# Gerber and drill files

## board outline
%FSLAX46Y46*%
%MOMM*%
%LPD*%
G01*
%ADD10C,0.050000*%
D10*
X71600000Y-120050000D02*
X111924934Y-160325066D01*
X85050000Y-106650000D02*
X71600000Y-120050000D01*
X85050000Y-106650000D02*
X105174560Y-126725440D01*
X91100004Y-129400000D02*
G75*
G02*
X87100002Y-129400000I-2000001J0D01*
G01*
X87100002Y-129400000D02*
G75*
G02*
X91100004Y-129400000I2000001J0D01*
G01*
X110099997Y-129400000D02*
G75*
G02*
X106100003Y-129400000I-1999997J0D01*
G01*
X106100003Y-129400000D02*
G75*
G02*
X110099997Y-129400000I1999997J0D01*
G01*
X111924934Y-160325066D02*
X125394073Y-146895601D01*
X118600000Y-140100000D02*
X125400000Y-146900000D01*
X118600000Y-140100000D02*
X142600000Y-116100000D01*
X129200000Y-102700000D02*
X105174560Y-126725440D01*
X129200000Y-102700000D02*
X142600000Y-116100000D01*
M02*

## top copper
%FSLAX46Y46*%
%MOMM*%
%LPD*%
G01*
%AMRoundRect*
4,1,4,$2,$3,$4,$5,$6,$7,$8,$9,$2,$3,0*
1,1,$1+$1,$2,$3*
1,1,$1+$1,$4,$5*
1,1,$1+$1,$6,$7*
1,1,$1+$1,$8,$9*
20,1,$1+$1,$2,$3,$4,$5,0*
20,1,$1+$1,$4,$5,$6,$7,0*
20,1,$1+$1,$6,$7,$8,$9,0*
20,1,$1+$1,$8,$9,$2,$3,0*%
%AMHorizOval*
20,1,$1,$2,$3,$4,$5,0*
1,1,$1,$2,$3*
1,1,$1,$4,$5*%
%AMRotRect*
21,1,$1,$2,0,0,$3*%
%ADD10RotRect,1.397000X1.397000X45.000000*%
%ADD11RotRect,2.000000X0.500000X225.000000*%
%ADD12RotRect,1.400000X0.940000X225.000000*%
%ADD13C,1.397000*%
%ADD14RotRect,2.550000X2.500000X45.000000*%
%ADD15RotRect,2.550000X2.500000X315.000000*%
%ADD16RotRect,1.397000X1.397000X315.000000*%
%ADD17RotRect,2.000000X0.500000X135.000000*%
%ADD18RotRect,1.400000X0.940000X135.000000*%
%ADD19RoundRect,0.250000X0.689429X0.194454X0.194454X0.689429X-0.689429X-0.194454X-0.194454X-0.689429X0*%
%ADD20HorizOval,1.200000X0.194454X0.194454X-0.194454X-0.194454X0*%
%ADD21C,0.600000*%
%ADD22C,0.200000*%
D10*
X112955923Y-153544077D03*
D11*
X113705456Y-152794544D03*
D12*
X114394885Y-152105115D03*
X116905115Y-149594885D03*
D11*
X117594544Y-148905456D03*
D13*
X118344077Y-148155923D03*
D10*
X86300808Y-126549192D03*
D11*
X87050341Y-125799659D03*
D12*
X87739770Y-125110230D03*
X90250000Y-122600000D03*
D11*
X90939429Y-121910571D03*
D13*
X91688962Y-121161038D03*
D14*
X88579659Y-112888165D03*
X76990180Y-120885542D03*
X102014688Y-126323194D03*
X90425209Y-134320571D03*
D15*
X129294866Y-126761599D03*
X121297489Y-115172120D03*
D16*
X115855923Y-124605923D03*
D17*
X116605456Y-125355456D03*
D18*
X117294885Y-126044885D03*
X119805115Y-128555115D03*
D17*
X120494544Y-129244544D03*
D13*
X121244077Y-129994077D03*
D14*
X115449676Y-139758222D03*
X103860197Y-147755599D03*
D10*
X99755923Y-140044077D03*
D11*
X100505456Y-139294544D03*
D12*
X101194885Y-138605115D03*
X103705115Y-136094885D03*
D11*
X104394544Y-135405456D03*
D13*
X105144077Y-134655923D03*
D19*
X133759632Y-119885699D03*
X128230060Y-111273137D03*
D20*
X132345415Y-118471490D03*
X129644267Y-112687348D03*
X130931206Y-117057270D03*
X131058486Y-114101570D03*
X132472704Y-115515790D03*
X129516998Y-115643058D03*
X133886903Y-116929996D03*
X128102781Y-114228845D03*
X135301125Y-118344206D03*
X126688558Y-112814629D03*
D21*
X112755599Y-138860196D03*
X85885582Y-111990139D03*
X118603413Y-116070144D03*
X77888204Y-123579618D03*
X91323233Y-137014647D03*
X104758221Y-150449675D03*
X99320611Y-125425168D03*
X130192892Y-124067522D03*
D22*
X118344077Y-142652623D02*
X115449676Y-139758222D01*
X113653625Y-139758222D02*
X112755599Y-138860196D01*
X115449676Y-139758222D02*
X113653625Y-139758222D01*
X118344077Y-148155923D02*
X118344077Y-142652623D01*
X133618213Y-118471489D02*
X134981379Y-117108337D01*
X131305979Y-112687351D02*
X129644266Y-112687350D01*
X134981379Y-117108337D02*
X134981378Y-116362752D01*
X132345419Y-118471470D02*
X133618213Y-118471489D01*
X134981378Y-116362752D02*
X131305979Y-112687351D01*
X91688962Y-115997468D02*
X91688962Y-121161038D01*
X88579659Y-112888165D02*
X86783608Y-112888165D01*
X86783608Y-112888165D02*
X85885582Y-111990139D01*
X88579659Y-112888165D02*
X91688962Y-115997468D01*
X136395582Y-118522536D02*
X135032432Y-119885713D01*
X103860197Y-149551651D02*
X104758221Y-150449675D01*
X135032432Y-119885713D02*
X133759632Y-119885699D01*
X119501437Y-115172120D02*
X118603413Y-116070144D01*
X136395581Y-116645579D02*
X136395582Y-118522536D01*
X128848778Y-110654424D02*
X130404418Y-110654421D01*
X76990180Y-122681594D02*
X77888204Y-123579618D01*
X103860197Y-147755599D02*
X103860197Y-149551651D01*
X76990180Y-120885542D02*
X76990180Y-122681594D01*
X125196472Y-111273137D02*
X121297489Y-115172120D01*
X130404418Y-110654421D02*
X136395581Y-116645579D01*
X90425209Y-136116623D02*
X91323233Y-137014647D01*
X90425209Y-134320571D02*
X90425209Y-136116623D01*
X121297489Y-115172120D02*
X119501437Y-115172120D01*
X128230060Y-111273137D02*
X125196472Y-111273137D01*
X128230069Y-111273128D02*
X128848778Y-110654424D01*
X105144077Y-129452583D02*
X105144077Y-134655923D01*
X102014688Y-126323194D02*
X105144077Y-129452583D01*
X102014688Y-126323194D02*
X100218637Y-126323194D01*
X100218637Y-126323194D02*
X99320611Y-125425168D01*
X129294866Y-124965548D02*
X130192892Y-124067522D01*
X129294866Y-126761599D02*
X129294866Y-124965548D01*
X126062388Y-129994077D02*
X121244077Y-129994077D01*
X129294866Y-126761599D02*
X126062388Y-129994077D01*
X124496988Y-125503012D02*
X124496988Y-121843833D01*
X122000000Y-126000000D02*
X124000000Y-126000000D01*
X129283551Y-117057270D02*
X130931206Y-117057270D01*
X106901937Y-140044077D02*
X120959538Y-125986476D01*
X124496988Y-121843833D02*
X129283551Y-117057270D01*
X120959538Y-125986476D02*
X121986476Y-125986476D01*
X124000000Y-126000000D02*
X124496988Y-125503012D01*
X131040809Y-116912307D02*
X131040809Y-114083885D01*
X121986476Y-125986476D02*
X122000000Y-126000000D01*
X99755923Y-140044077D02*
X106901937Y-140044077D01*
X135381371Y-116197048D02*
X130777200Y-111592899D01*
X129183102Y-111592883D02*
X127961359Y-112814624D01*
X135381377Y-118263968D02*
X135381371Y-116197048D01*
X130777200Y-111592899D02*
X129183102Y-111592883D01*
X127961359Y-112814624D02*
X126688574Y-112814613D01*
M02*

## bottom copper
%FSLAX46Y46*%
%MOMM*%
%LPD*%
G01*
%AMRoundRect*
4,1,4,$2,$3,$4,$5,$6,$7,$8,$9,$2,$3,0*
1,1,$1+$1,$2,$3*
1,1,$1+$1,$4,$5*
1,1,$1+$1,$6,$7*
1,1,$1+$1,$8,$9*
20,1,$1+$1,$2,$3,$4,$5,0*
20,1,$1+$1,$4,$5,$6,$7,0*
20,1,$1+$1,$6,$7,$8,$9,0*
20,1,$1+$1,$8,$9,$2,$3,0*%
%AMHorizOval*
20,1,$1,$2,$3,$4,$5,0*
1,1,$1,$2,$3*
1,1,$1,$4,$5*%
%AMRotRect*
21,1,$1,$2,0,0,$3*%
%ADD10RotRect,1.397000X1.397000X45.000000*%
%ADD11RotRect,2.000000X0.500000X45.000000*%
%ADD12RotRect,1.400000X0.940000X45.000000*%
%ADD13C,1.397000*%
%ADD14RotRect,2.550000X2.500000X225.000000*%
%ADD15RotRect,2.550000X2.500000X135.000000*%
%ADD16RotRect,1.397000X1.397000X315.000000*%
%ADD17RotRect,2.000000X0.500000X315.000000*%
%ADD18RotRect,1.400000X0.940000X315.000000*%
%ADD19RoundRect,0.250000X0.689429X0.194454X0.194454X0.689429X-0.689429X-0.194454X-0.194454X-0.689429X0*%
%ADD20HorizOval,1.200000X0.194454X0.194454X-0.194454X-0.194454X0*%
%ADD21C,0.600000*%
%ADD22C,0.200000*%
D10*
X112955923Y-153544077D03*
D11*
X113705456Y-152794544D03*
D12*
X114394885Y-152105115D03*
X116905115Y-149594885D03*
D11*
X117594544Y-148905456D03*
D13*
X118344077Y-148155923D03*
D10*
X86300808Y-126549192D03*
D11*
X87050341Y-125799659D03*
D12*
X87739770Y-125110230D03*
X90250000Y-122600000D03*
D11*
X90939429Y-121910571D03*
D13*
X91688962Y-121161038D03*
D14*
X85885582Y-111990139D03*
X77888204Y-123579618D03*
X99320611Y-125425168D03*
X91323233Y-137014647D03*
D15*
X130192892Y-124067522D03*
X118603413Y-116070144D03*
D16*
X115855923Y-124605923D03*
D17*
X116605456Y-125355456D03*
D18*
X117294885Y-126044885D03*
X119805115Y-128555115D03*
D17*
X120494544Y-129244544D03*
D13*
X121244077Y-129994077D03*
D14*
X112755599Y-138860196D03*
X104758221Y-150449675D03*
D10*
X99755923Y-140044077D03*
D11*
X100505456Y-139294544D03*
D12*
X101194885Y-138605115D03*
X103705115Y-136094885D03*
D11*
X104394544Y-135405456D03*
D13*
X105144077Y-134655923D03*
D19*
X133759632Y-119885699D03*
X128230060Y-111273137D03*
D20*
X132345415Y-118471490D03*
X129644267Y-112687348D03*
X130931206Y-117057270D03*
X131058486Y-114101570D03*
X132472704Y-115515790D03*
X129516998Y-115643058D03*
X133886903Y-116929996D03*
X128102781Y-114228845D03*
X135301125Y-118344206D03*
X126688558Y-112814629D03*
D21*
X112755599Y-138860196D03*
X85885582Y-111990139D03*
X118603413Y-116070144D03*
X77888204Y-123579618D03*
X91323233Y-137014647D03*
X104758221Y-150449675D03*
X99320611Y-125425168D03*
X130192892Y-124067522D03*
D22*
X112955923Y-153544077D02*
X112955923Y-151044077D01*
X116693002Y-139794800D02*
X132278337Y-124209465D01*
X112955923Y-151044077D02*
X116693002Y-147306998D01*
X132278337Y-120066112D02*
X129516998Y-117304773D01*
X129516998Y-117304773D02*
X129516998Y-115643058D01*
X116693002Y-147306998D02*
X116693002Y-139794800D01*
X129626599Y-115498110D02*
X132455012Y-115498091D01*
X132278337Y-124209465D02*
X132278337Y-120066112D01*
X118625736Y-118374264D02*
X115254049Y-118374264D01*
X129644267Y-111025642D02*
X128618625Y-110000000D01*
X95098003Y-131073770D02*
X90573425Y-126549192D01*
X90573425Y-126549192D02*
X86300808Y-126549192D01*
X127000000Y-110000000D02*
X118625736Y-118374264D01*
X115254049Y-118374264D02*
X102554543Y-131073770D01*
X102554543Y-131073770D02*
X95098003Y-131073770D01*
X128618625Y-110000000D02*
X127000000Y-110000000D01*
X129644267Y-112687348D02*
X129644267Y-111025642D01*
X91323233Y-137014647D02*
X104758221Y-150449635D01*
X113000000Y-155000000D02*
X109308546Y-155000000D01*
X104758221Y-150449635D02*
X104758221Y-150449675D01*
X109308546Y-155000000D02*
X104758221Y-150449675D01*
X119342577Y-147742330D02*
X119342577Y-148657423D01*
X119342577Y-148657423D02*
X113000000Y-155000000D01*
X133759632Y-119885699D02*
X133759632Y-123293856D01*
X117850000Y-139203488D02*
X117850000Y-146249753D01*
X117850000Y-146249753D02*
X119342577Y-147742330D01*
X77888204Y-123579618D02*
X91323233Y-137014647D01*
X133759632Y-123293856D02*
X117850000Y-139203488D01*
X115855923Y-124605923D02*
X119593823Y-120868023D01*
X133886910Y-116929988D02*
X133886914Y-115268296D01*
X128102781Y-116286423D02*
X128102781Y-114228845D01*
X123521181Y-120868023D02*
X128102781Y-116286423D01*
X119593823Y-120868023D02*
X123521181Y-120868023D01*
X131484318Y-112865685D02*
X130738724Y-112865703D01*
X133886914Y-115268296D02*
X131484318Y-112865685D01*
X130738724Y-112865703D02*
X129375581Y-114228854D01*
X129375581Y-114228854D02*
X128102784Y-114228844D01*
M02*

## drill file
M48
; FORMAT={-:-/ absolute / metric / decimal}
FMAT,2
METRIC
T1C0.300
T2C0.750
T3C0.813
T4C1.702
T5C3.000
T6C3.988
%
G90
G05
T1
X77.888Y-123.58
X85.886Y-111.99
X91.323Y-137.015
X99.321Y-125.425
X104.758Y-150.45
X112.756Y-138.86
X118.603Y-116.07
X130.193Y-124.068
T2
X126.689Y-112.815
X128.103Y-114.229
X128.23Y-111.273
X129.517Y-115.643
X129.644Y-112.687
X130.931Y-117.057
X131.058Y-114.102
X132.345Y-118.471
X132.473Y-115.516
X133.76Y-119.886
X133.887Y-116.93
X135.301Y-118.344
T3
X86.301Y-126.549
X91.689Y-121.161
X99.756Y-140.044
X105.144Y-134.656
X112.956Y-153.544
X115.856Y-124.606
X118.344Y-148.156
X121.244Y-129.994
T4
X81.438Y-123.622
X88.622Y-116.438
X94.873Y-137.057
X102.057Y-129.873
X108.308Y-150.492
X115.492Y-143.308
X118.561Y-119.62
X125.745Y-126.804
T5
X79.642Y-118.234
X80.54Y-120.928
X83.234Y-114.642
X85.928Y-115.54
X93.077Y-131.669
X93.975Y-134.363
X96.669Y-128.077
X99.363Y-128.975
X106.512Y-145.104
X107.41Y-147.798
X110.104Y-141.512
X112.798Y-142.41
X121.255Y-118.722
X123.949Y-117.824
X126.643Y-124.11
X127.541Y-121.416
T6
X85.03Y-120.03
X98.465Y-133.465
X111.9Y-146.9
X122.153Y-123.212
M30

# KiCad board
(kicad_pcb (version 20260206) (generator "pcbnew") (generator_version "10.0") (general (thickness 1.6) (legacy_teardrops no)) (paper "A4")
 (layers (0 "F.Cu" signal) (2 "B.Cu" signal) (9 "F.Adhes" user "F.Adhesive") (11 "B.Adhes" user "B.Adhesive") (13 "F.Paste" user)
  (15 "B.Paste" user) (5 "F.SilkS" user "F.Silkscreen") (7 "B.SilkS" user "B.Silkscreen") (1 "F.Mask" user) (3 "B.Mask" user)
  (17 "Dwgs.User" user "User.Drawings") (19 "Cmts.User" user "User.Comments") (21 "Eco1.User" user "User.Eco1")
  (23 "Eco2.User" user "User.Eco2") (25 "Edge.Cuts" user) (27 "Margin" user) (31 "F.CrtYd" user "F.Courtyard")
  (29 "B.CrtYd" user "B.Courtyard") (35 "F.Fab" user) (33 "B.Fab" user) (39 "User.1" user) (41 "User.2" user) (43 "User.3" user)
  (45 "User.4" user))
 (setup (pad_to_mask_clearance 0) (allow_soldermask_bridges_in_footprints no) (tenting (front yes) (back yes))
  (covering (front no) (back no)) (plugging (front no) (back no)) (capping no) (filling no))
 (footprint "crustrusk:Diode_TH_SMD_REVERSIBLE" (layer "F.Cu") (at 115.65 150.85 45)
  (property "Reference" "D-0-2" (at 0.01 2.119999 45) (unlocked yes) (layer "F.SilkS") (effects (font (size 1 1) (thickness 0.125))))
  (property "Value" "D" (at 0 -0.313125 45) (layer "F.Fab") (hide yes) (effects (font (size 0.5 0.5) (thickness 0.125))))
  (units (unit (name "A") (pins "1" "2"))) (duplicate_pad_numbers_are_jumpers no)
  (pad "1" thru_hole rect (at -3.81 0 45) (size 1.397 1.397) (drill 0.8128) (layers "*.Cu" "*.Mask") (remove_unused_layers no)
   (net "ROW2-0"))
  (pad "1" smd rect (at -2.75 0 225) (size 2 0.5) (layers "F.Cu") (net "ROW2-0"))
  (pad "1" smd rect (at -2.75 0 45) (size 2 0.5) (layers "B.Cu") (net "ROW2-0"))
  (pad "1" smd rect (at -1.775001 0 225) (size 1.4 0.94) (layers "F.Cu" "F.Mask" "F.Paste") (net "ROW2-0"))
  (pad "1" smd rect (at -1.775001 0 45) (size 1.4 0.94) (layers "B.Cu" "B.Mask" "B.Paste") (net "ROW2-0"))
  (pad "2" smd rect (at 1.775001 0 225) (size 1.4 0.94) (layers "F.Cu" "F.Mask" "F.Paste") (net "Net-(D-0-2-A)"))
  (pad "2" smd rect (at 1.775001 0 45) (size 1.4 0.94) (layers "B.Cu" "B.Mask" "B.Paste") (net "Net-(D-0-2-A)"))
  (pad "2" smd rect (at 2.75 0 225) (size 2 0.5) (layers "F.Cu") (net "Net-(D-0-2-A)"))
  (pad "2" smd rect (at 2.75 0 45) (size 2 0.5) (layers "B.Cu") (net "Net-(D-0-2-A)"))
  (pad "2" thru_hole circle (at 3.81 0 45) (size 1.397 1.397) (drill 0.8128) (layers "*.Cu" "*.Mask") (remove_unused_layers no)
   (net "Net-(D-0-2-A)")))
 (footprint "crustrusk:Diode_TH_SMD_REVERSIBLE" (layer "F.Cu") (at 88.994885 123.855115 45)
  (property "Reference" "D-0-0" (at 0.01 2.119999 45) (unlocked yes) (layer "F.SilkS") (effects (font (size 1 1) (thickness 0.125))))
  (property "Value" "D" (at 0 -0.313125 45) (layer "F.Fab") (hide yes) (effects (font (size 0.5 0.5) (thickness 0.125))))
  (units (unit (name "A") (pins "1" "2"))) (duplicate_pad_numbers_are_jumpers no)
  (pad "1" thru_hole rect (at -3.81 0 45) (size 1.397 1.397) (drill 0.8128) (layers "*.Cu" "*.Mask") (remove_unused_layers no)
   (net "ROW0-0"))
  (pad "1" smd rect (at -2.75 0 225) (size 2 0.5) (layers "F.Cu") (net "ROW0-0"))
  (pad "1" smd rect (at -2.75 0 45) (size 2 0.5) (layers "B.Cu") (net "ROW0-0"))
  (pad "1" smd rect (at -1.775001 0 225) (size 1.4 0.94) (layers "F.Cu" "F.Mask" "F.Paste") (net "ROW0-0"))
  (pad "1" smd rect (at -1.775001 0 45) (size 1.4 0.94) (layers "B.Cu" "B.Mask" "B.Paste") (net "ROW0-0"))
  (pad "2" smd rect (at 1.775001 0 225) (size 1.4 0.94) (layers "F.Cu" "F.Mask" "F.Paste") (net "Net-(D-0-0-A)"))
  (pad "2" smd rect (at 1.775001 0 45) (size 1.4 0.94) (layers "B.Cu" "B.Mask" "B.Paste") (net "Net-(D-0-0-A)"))
  (pad "2" smd rect (at 2.75 0 225) (size 2 0.5) (layers "F.Cu") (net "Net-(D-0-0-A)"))
  (pad "2" smd rect (at 2.75 0 45) (size 2 0.5) (layers "B.Cu") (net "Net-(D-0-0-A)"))
  (pad "2" thru_hole circle (at 3.81 0 45) (size 1.397 1.397) (drill 0.8128) (layers "*.Cu" "*.Mask") (remove_unused_layers no)
   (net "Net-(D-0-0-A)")))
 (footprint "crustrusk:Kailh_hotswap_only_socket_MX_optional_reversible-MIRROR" (layer "F.Cu") (at 85.029983 120.029943 45)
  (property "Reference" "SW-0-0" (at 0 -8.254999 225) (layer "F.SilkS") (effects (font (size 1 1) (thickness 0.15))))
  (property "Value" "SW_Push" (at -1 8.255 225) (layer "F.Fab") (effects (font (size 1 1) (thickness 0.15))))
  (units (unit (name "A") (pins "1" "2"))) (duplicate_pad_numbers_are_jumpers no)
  (pad "" np_thru_hole circle (at -5.079999 0 45) (size 1.7018 1.7018) (drill 1.7018) (layers "*.Cu" "*.Mask"))
  (pad "" np_thru_hole circle (at -3.81 -2.54 225) (size 3 3) (drill 3) (layers "*.Cu" "*.Mask"))
  (pad "" np_thru_hole circle (at -2.54 -5.079998 45) (size 3 3) (drill 3) (layers "*.Cu" "*.Mask"))
  (pad "" np_thru_hole circle (at 0 0 45) (size 3.9878 3.9878) (drill 3.9878) (layers "*.Cu" "*.Mask"))
  (pad "" np_thru_hole circle (at 2.540002 -5.080001 225) (size 3 3) (drill 3) (layers "*.Cu" "*.Mask"))
  (pad "" np_thru_hole circle (at 3.81 -2.54 45) (size 3 3) (drill 3) (layers "*.Cu" "*.Mask"))
  (pad "" np_thru_hole circle (at 5.079999 0 45) (size 1.7018 1.7018) (drill 1.7018) (layers "*.Cu" "*.Mask"))
  (pad "1" smd rect (at 6.29 -5.08 225) (size 2.55 2.5) (layers "B.Cu" "B.Mask" "B.Paste") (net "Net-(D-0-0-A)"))
  (pad "1" smd rect (at 7.56 -2.54 45) (size 2.55 2.5) (layers "F.Cu" "F.Mask" "F.Paste") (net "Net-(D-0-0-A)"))
  (pad "2" smd rect (at -7.56 -2.540001 225) (size 2.55 2.5) (layers "B.Cu" "B.Mask" "B.Paste") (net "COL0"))
  (pad "2" smd rect (at -6.289999 -5.079999 45) (size 2.55 2.5) (layers "F.Cu" "F.Mask" "F.Paste") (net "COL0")))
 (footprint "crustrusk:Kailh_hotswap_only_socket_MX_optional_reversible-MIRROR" (layer "F.Cu") (at 98.465012 133.464972 45)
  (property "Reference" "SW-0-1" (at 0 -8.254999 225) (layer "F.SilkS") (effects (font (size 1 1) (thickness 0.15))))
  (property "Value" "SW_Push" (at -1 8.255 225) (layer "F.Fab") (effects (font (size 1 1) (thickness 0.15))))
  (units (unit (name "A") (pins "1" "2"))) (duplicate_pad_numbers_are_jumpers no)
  (pad "" np_thru_hole circle (at -5.079999 0 45) (size 1.7018 1.7018) (drill 1.7018) (layers "*.Cu" "*.Mask"))
  (pad "" np_thru_hole circle (at -3.81 -2.54 225) (size 3 3) (drill 3) (layers "*.Cu" "*.Mask"))
  (pad "" np_thru_hole circle (at -2.54 -5.079998 45) (size 3 3) (drill 3) (layers "*.Cu" "*.Mask"))
  (pad "" np_thru_hole circle (at 0 0 45) (size 3.9878 3.9878) (drill 3.9878) (layers "*.Cu" "*.Mask"))
  (pad "" np_thru_hole circle (at 2.540002 -5.080001 225) (size 3 3) (drill 3) (layers "*.Cu" "*.Mask"))
  (pad "" np_thru_hole circle (at 3.81 -2.54 45) (size 3 3) (drill 3) (layers "*.Cu" "*.Mask"))
  (pad "" np_thru_hole circle (at 5.079999 0 45) (size 1.7018 1.7018) (drill 1.7018) (layers "*.Cu" "*.Mask"))
  (pad "1" smd rect (at 6.29 -5.08 225) (size 2.55 2.5) (layers "B.Cu" "B.Mask" "B.Paste") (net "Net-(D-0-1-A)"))
  (pad "1" smd rect (at 7.56 -2.54 45) (size 2.55 2.5) (layers "F.Cu" "F.Mask" "F.Paste") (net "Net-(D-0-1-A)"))
  (pad "2" smd rect (at -7.56 -2.540001 225) (size 2.55 2.5) (layers "B.Cu" "B.Mask" "B.Paste") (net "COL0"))
  (pad "2" smd rect (at -6.289999 -5.079999 45) (size 2.55 2.5) (layers "F.Cu" "F.Mask" "F.Paste") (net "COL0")))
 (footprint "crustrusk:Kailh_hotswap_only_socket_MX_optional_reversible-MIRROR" (layer "F.Cu") (at 122.153088 123.211923 -45)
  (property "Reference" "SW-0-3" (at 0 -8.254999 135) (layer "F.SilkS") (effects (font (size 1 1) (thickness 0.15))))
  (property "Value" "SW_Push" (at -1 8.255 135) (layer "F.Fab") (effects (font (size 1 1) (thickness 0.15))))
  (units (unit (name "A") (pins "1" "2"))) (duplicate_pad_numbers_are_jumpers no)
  (pad "" np_thru_hole circle (at -5.079999 0 315) (size 1.7018 1.7018) (drill 1.7018) (layers "*.Cu" "*.Mask"))
  (pad "" np_thru_hole circle (at -3.81 -2.54 135) (size 3 3) (drill 3) (layers "*.Cu" "*.Mask"))
  (pad "" np_thru_hole circle (at -2.54 -5.079998 315) (size 3 3) (drill 3) (layers "*.Cu" "*.Mask"))
  (pad "" np_thru_hole circle (at 0 0 315) (size 3.9878 3.9878) (drill 3.9878) (layers "*.Cu" "*.Mask"))
  (pad "" np_thru_hole circle (at 2.540002 -5.080001 135) (size 3 3) (drill 3) (layers "*.Cu" "*.Mask"))
  (pad "" np_thru_hole circle (at 3.81 -2.54 315) (size 3 3) (drill 3) (layers "*.Cu" "*.Mask"))
  (pad "" np_thru_hole circle (at 5.079999 0 315) (size 1.7018 1.7018) (drill 1.7018) (layers "*.Cu" "*.Mask"))
  (pad "1" smd rect (at 6.29 -5.08 135) (size 2.55 2.5) (layers "B.Cu" "B.Mask" "B.Paste") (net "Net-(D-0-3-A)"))
  (pad "1" smd rect (at 7.56 -2.54 315) (size 2.55 2.5) (layers "F.Cu" "F.Mask" "F.Paste") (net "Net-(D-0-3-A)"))
  (pad "2" smd rect (at -7.56 -2.540001 135) (size 2.55 2.5) (layers "B.Cu" "B.Mask" "B.Paste") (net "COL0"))
  (pad "2" smd rect (at -6.289999 -5.079999 315) (size 2.55 2.5) (layers "F.Cu" "F.Mask" "F.Paste") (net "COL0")))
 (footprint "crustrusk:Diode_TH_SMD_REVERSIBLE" (layer "F.Cu") (at 118.55 127.3 -45)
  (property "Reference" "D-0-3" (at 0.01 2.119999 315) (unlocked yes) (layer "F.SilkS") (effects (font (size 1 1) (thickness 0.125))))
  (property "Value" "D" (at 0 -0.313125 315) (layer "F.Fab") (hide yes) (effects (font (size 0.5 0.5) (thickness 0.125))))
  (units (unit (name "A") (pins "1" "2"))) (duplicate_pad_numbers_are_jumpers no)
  (pad "1" thru_hole rect (at -3.81 0 315) (size 1.397 1.397) (drill 0.8128) (layers "*.Cu" "*.Mask") (remove_unused_layers no)
   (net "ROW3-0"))
  (pad "1" smd rect (at -2.75 0 135) (size 2 0.5) (layers "F.Cu") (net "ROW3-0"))
  (pad "1" smd rect (at -2.75 0 315) (size 2 0.5) (layers "B.Cu") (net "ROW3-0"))
  (pad "1" smd rect (at -1.775001 0 135) (size 1.4 0.94) (layers "F.Cu" "F.Mask" "F.Paste") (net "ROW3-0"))
  (pad "1" smd rect (at -1.775001 0 315) (size 1.4 0.94) (layers "B.Cu" "B.Mask" "B.Paste") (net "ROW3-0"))
  (pad "2" smd rect (at 1.775001 0 135) (size 1.4 0.94) (layers "F.Cu" "F.Mask" "F.Paste") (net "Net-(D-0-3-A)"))
  (pad "2" smd rect (at 1.775001 0 315) (size 1.4 0.94) (layers "B.Cu" "B.Mask" "B.Paste") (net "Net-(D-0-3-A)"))
  (pad "2" smd rect (at 2.75 0 135) (size 2 0.5) (layers "F.Cu") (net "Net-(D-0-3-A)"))
  (pad "2" smd rect (at 2.75 0 315) (size 2 0.5) (layers "B.Cu") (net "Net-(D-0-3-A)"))
  (pad "2" thru_hole circle (at 3.81 0 315) (size 1.397 1.397) (drill 0.8128) (layers "*.Cu" "*.Mask") (remove_unused_layers no)
   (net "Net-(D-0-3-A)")))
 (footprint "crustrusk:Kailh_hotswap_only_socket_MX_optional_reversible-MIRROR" (layer "F.Cu") (at 111.9 146.9 45)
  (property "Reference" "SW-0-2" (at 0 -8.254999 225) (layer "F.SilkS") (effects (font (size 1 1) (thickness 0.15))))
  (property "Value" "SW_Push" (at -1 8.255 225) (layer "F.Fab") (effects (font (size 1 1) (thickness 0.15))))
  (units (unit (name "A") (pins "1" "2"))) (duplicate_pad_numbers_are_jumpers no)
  (pad "" np_thru_hole circle (at -5.079999 0 45) (size 1.7018 1.7018) (drill 1.7018) (layers "*.Cu" "*.Mask"))
  (pad "" np_thru_hole circle (at -3.81 -2.54 225) (size 3 3) (drill 3) (layers "*.Cu" "*.Mask"))
  (pad "" np_thru_hole circle (at -2.54 -5.079998 45) (size 3 3) (drill 3) (layers "*.Cu" "*.Mask"))
  (pad "" np_thru_hole circle (at 0 0 45) (size 3.9878 3.9878) (drill 3.9878) (layers "*.Cu" "*.Mask"))
  (pad "" np_thru_hole circle (at 2.540002 -5.080001 225) (size 3 3) (drill 3) (layers "*.Cu" "*.Mask"))
  (pad "" np_thru_hole circle (at 3.81 -2.54 45) (size 3 3) (drill 3) (layers "*.Cu" "*.Mask"))
  (pad "" np_thru_hole circle (at 5.079999 0 45) (size 1.7018 1.7018) (drill 1.7018) (layers "*.Cu" "*.Mask"))
  (pad "1" smd rect (at 6.29 -5.08 225) (size 2.55 2.5) (layers "B.Cu" "B.Mask" "B.Paste") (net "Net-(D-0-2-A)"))
  (pad "1" smd rect (at 7.56 -2.54 45) (size 2.55 2.5) (layers "F.Cu" "F.Mask" "F.Paste") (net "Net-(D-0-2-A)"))
  (pad "2" smd rect (at -7.56 -2.540001 225) (size 2.55 2.5) (layers "B.Cu" "B.Mask" "B.Paste") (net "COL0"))
  (pad "2" smd rect (at -6.289999 -5.079999 45) (size 2.55 2.5) (layers "F.Cu" "F.Mask" "F.Paste") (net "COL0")))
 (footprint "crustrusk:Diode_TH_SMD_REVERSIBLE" (layer "F.Cu") (at 102.45 137.35 45)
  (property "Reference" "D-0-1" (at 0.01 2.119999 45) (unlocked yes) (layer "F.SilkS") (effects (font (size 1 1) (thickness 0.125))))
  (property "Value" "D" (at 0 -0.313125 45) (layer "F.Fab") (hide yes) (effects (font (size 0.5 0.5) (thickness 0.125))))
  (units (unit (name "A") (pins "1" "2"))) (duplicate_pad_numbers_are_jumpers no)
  (pad "1" thru_hole rect (at -3.81 0 45) (size 1.397 1.397) (drill 0.8128) (layers "*.Cu" "*.Mask") (remove_unused_layers no)
   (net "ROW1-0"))
  (pad "1" smd rect (at -2.75 0 225) (size 2 0.5) (layers "F.Cu") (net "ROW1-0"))
  (pad "1" smd rect (at -2.75 0 45) (size 2 0.5) (layers "B.Cu") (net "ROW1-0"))
  (pad "1" smd rect (at -1.775001 0 225) (size 1.4 0.94) (layers "F.Cu" "F.Mask" "F.Paste") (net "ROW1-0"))
  (pad "1" smd rect (at -1.775001 0 45) (size 1.4 0.94) (layers "B.Cu" "B.Mask" "B.Paste") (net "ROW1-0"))
  (pad "2" smd rect (at 1.775001 0 225) (size 1.4 0.94) (layers "F.Cu" "F.Mask" "F.Paste") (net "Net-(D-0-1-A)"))
  (pad "2" smd rect (at 1.775001 0 45) (size 1.4 0.94) (layers "B.Cu" "B.Mask" "B.Paste") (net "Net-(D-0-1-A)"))
  (pad "2" smd rect (at 2.75 0 225) (size 2 0.5) (layers "F.Cu") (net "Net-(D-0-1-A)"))
  (pad "2" smd rect (at 2.75 0 45) (size 2 0.5) (layers "B.Cu") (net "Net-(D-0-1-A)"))
  (pad "2" thru_hole circle (at 3.81 0 45) (size 1.397 1.397) (drill 0.8128) (layers "*.Cu" "*.Mask") (remove_unused_layers no)
   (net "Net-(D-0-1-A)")))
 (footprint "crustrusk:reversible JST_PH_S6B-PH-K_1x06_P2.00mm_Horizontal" (layer "F.Cu") (at 133.759632 119.885699 135)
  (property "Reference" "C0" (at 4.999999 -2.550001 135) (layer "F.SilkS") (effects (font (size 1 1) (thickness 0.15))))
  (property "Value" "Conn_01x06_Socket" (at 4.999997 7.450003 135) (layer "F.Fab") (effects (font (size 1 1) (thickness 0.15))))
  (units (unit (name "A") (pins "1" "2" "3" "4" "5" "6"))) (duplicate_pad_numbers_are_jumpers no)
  (pad "1" thru_hole roundrect (at 0 0 135) (size 1.2 1.75) (drill 0.75) (layers "*.Cu" "*.Mask") (remove_unused_layers no)
   (roundrect_rratio 0.208333) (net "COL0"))
  (pad "1" thru_hole roundrect (at 9.999999 2.180003 135) (size 1.2 1.75) (drill 0.75) (layers "*.Cu" "*.Mask") (remove_unused_layers no)
   (roundrect_rratio 0.208333) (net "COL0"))
  (pad "2" thru_hole oval (at 1.999999 -0.000006 135) (size 1.2 1.75) (drill 0.75) (layers "*.Cu" "*.Mask") (remove_unused_layers no)
   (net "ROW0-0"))
  (pad "2" thru_hole oval (at 8.000005 2.18 135) (size 1.2 1.75) (drill 0.75) (layers "*.Cu" "*.Mask") (remove_unused_layers no)
   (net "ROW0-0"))
  (pad "3" thru_hole oval (at 4.000001 0.000002 135) (size 1.2 1.75) (drill 0.75) (layers "*.Cu" "*.Mask") (remove_unused_layers no)
   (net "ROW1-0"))
  (pad "3" thru_hole oval (at 5.999995 2.179998 135) (size 1.2 1.75) (drill 0.75) (layers "*.Cu" "*.Mask") (remove_unused_layers no)
   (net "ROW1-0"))
  (pad "4" thru_hole oval (at 3.999988 2.179997 135) (size 1.2 1.75) (drill 0.75) (layers "*.Cu" "*.Mask") (remove_unused_layers no)
   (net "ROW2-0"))
  (pad "4" thru_hole oval (at 5.999995 0.000005 135) (size 1.2 1.75) (drill 0.75) (layers "*.Cu" "*.Mask") (remove_unused_layers no)
   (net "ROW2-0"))
  (pad "5" thru_hole oval (at 2.000003 2.179992 135) (size 1.2 1.75) (drill 0.75) (layers "*.Cu" "*.Mask") (remove_unused_layers no)
   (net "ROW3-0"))
  (pad "5" thru_hole oval (at 7.999998 0.000002 135) (size 1.2 1.75) (drill 0.75) (layers "*.Cu" "*.Mask") (remove_unused_layers no)
   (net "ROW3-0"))
  (pad "6" thru_hole oval (at 0 2.18 135) (size 1.2 1.75) (drill 0.75) (layers "*.Cu" "*.Mask") (remove_unused_layers no) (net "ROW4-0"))
  (pad "6" thru_hole oval (at 10.000006 -0.000003 135) (size 1.2 1.75) (drill 0.75) (layers "*.Cu" "*.Mask") (remove_unused_layers no)
   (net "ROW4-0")))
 (gr_line (start 71.6 120.05) (end 111.924934 160.325066) (stroke (width 0.05) (type default)) (layer "Edge.Cuts"))
 (gr_line (start 85.05 106.65) (end 71.6 120.05) (stroke (width 0.05) (type default)) (layer "Edge.Cuts"))
 (gr_line (start 85.05 106.65) (end 105.17456 126.72544) (stroke (width 0.05) (type default)) (layer "Edge.Cuts"))
 (gr_circle (center 89.100003 129.4) (end 87.100002 129.4) (stroke (width 0.05) (type default)) (fill no) (layer "Edge.Cuts"))
 (gr_circle (center 108.1 129.4) (end 106.100003 129.4) (stroke (width 0.05) (type default)) (fill no) (layer "Edge.Cuts"))
 (gr_line (start 111.924934 160.325066) (end 125.394073 146.895601) (stroke (width 0.05) (type default)) (layer "Edge.Cuts"))
 (gr_line (start 118.6 140.1) (end 125.4 146.9) (stroke (width 0.05) (type default)) (layer "Edge.Cuts"))
 (gr_line (start 118.6 140.1) (end 142.6 116.1) (stroke (width 0.05) (type default)) (layer "Edge.Cuts"))
 (gr_line (start 129.2 102.7) (end 105.17456 126.72544) (stroke (width 0.05) (type default)) (layer "Edge.Cuts"))
 (gr_line (start 129.2 102.7) (end 142.6 116.1) (stroke (width 0.05) (type default)) (layer "Edge.Cuts"))
 (segment (start 112.955923 153.544077) (end 112.955923 151.044077) (width 0.2) (layer "B.Cu") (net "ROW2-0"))
 (segment (start 116.693002 139.7948) (end 132.278337 124.209465) (width 0.2) (layer "B.Cu") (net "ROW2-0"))
 (segment (start 112.955923 151.044077) (end 116.693002 147.306998) (width 0.2) (layer "B.Cu") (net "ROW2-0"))
 (segment (start 132.278337 120.066112) (end 129.516998 117.304773) (width 0.2) (layer "B.Cu") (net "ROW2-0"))
 (segment (start 129.516998 117.304773) (end 129.516998 115.643058) (width 0.2) (layer "B.Cu") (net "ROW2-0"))
 (segment (start 116.693002 147.306998) (end 116.693002 139.7948) (width 0.2) (layer "B.Cu") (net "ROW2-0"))
 (segment (start 129.626599 115.49811) (end 132.455012 115.498091) (width 0.2) (layer "B.Cu") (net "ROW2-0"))
 (segment (start 132.278337 124.209465) (end 132.278337 120.066112) (width 0.2) (layer "B.Cu") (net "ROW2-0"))
 (segment (start 118.344077 142.652623) (end 115.449676 139.758222) (width 0.2) (layer "F.Cu") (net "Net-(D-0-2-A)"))
 (segment (start 113.653625 139.758222) (end 112.755599 138.860196) (width 0.2) (layer "F.Cu") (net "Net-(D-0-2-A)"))
 (segment (start 115.449676 139.758222) (end 113.653625 139.758222) (width 0.2) (layer "F.Cu") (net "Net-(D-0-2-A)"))
 (segment (start 118.344077 148.155923) (end 118.344077 142.652623) (width 0.2) (layer "F.Cu") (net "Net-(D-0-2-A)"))
 (via (at 112.755599 138.860196) (size 0.6) (drill 0.3) (layers "F.Cu" "B.Cu") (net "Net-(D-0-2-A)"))
 (segment (start 133.618213 118.471489) (end 134.981379 117.108337) (width 0.2) (layer "F.Cu") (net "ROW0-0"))
 (segment (start 131.305979 112.687351) (end 129.644266 112.68735) (width 0.2) (layer "F.Cu") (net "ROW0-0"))
 (segment (start 134.981379 117.108337) (end 134.981378 116.362752) (width 0.2) (layer "F.Cu") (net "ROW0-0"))
 (segment (start 132.345419 118.47147) (end 133.618213 118.471489) (width 0.2) (layer "F.Cu") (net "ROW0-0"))
 (segment (start 134.981378 116.362752) (end 131.305979 112.687351) (width 0.2) (layer "F.Cu") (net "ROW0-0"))
 (segment (start 118.625736 118.374264) (end 115.254049 118.374264) (width 0.2) (layer "B.Cu") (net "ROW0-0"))
 (segment (start 129.644267 111.025642) (end 128.618625 110) (width 0.2) (layer "B.Cu") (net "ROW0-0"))
 (segment (start 95.098003 131.07377) (end 90.573425 126.549192) (width 0.2) (layer "B.Cu") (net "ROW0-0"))
 (segment (start 90.573425 126.549192) (end 86.300808 126.549192) (width 0.2) (layer "B.Cu") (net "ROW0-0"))
 (segment (start 127 110) (end 118.625736 118.374264) (width 0.2) (layer "B.Cu") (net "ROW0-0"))
 (segment (start 115.254049 118.374264) (end 102.554543 131.07377) (width 0.2) (layer "B.Cu") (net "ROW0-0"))
 (segment (start 102.554543 131.07377) (end 95.098003 131.07377) (width 0.2) (layer "B.Cu") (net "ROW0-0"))
 (segment (start 128.618625 110) (end 127 110) (width 0.2) (layer "B.Cu") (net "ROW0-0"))
 (segment (start 129.644267 112.687348) (end 129.644267 111.025642) (width 0.2) (layer "B.Cu") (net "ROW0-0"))
 (segment (start 91.688962 115.997468) (end 91.688962 121.161038) (width 0.2) (layer "F.Cu") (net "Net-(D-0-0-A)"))
 (segment (start 88.579659 112.888165) (end 86.783608 112.888165) (width 0.2) (layer "F.Cu") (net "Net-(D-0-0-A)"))
 (segment (start 86.783608 112.888165) (end 85.885582 111.990139) (width 0.2) (layer "F.Cu") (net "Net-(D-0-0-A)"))
 (segment (start 88.579659 112.888165) (end 91.688962 115.997468) (width 0.2) (layer "F.Cu") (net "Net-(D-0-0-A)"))
 (via (at 85.885582 111.990139) (size 0.6) (drill 0.3) (layers "F.Cu" "B.Cu") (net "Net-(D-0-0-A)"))
 (segment (start 136.395582 118.522536) (end 135.032432 119.885713) (width 0.2) (layer "F.Cu") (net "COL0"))
 (segment (start 103.860197 149.551651) (end 104.758221 150.449675) (width 0.2) (layer "F.Cu") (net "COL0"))
 (segment (start 135.032432 119.885713) (end 133.759632 119.885699) (width 0.2) (layer "F.Cu") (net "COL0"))
 (segment (start 119.501437 115.17212) (end 118.603413 116.070144) (width 0.2) (layer "F.Cu") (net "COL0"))
 (segment (start 136.395581 116.645579) (end 136.395582 118.522536) (width 0.2) (layer "F.Cu") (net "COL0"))
 (segment (start 128.848778 110.654424) (end 130.404418 110.654421) (width 0.2) (layer "F.Cu") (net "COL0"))
 (segment (start 76.99018 122.681594) (end 77.888204 123.579618) (width 0.2) (layer "F.Cu") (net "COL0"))
 (segment (start 103.860197 147.755599) (end 103.860197 149.551651) (width 0.2) (layer "F.Cu") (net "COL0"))
 (segment (start 76.99018 120.885542) (end 76.99018 122.681594) (width 0.2) (layer "F.Cu") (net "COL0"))
 (segment (start 125.196472 111.273137) (end 121.297489 115.17212) (width 0.2) (layer "F.Cu") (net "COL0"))
 (segment (start 130.404418 110.654421) (end 136.395581 116.645579) (width 0.2) (layer "F.Cu") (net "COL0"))
 (segment (start 90.425209 136.116623) (end 91.323233 137.014647) (width 0.2) (layer "F.Cu") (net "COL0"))
 (segment (start 90.425209 134.320571) (end 90.425209 136.116623) (width 0.2) (layer "F.Cu") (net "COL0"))
 (segment (start 121.297489 115.17212) (end 119.501437 115.17212) (width 0.2) (layer "F.Cu") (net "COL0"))
 (segment (start 128.23006 111.273137) (end 125.196472 111.273137) (width 0.2) (layer "F.Cu") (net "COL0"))
 (segment (start 128.230069 111.273128) (end 128.848778 110.654424) (width 0.2) (layer "F.Cu") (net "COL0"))
 (via (at 118.603413 116.070144) (size 0.6) (drill 0.3) (layers "F.Cu" "B.Cu") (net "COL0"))
 (via (at 77.888204 123.579618) (size 0.6) (drill 0.3) (layers "F.Cu" "B.Cu") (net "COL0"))
 (via (at 91.323233 137.014647) (size 0.6) (drill 0.3) (layers "F.Cu" "B.Cu") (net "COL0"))
 (via (at 104.758221 150.449675) (size 0.6) (drill 0.3) (layers "F.Cu" "B.Cu") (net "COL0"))
 (segment (start 91.323233 137.014647) (end 104.758221 150.449635) (width 0.2) (layer "B.Cu") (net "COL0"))
 (segment (start 113 155) (end 109.308546 155) (width 0.2) (layer "B.Cu") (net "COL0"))
 (segment (start 104.758221 150.449635) (end 104.758221 150.449675) (width 0.2) (layer "B.Cu") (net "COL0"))
 (segment (start 109.308546 155) (end 104.758221 150.449675) (width 0.2) (layer "B.Cu") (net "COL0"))
 (segment (start 119.342577 147.74233) (end 119.342577 148.657423) (width 0.2) (layer "B.Cu") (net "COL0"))
 (segment (start 119.342577 148.657423) (end 113 155) (width 0.2) (layer "B.Cu") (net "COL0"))
 (segment (start 133.759632 119.885699) (end 133.759632 123.293856) (width 0.2) (layer "B.Cu") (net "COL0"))
 (segment (start 117.85 139.203488) (end 117.85 146.249753) (width 0.2) (layer "B.Cu") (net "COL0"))
 (segment (start 117.85 146.249753) (end 119.342577 147.74233) (width 0.2) (layer "B.Cu") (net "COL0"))
 (segment (start 77.888204 123.579618) (end 91.323233 137.014647) (width 0.2) (layer "B.Cu") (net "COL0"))
 (segment (start 133.759632 123.293856) (end 117.85 139.203488) (width 0.2) (layer "B.Cu") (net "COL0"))
 (segment (start 105.144077 129.452583) (end 105.144077 134.655923) (width 0.2) (layer "F.Cu") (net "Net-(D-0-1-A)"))
 (segment (start 102.014688 126.323194) (end 105.144077 129.452583) (width 0.2) (layer "F.Cu") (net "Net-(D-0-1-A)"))
 (segment (start 102.014688 126.323194) (end 100.218637 126.323194) (width 0.2) (layer "F.Cu") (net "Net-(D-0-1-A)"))
 (segment (start 100.218637 126.323194) (end 99.320611 125.425168) (width 0.2) (layer "F.Cu") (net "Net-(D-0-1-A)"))
 (via (at 99.320611 125.425168) (size 0.6) (drill 0.3) (layers "F.Cu" "B.Cu") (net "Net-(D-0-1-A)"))
 (segment (start 115.855923 124.605923) (end 119.593823 120.868023) (width 0.2) (layer "B.Cu") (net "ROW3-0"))
 (segment (start 133.88691 116.929988) (end 133.886914 115.268296) (width 0.2) (layer "B.Cu") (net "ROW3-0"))
 (segment (start 128.102781 116.286423) (end 128.102781 114.228845) (width 0.2) (layer "B.Cu") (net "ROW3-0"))
 (segment (start 123.521181 120.868023) (end 128.102781 116.286423) (width 0.2) (layer "B.Cu") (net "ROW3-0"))
 (segment (start 119.593823 120.868023) (end 123.521181 120.868023) (width 0.2) (layer "B.Cu") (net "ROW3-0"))
 (segment (start 131.484318 112.865685) (end 130.738724 112.865703) (width 0.2) (layer "B.Cu") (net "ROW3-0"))
 (segment (start 133.886914 115.268296) (end 131.484318 112.865685) (width 0.2) (layer "B.Cu") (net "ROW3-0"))
 (segment (start 130.738724 112.865703) (end 129.375581 114.228854) (width 0.2) (layer "B.Cu") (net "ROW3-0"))
 (segment (start 129.375581 114.228854) (end 128.102784 114.228844) (width 0.2) (layer "B.Cu") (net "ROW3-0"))
 (segment (start 129.294866 124.965548) (end 130.192892 124.067522) (width 0.2) (layer "F.Cu") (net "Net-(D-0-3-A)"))
 (segment (start 129.294866 126.761599) (end 129.294866 124.965548) (width 0.2) (layer "F.Cu") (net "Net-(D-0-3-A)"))
 (segment (start 126.062388 129.994077) (end 121.244077 129.994077) (width 0.2) (layer "F.Cu") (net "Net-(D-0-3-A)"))
 (segment (start 129.294866 126.761599) (end 126.062388 129.994077) (width 0.2) (layer "F.Cu") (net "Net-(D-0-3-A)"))
 (via (at 130.192892 124.067522) (size 0.6) (drill 0.3) (layers "F.Cu" "B.Cu") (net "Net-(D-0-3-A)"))
 (segment (start 124.496988 125.503012) (end 124.496988 121.843833) (width 0.2) (layer "F.Cu") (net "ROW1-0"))
 (segment (start 122 126) (end 124 126) (width 0.2) (layer "F.Cu") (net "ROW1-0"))
 (segment (start 129.283551 117.05727) (end 130.931206 117.05727) (width 0.2) (layer "F.Cu") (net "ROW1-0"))
 (segment (start 106.901937 140.044077) (end 120.959538 125.986476) (width 0.2) (layer "F.Cu") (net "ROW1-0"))
 (segment (start 124.496988 121.843833) (end 129.283551 117.05727) (width 0.2) (layer "F.Cu") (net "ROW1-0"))
 (segment (start 120.959538 125.986476) (end 121.986476 125.986476) (width 0.2) (layer "F.Cu") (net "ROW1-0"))
 (segment (start 124 126) (end 124.496988 125.503012) (width 0.2) (layer "F.Cu") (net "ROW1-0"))
 (segment (start 131.040809 116.912307) (end 131.040809 114.083885) (width 0.2) (layer "F.Cu") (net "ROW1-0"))
 (segment (start 121.986476 125.986476) (end 122 126) (width 0.2) (layer "F.Cu") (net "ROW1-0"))
 (segment (start 99.755923 140.044077) (end 106.901937 140.044077) (width 0.2) (layer "F.Cu") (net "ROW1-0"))
 (segment (start 135.381371 116.197048) (end 130.7772 111.592899) (width 0.2) (layer "F.Cu") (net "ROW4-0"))
 (segment (start 129.183102 111.592883) (end 127.961359 112.814624) (width 0.2) (layer "F.Cu") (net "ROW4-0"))
 (segment (start 135.381377 118.263968) (end 135.381371 116.197048) (width 0.2) (layer "F.Cu") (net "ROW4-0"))
 (segment (start 130.7772 111.592899) (end 129.183102 111.592883) (width 0.2) (layer "F.Cu") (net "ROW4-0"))
 (segment (start 127.961359 112.814624) (end 126.688574 112.814613) (width 0.2) (layer "F.Cu") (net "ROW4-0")))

